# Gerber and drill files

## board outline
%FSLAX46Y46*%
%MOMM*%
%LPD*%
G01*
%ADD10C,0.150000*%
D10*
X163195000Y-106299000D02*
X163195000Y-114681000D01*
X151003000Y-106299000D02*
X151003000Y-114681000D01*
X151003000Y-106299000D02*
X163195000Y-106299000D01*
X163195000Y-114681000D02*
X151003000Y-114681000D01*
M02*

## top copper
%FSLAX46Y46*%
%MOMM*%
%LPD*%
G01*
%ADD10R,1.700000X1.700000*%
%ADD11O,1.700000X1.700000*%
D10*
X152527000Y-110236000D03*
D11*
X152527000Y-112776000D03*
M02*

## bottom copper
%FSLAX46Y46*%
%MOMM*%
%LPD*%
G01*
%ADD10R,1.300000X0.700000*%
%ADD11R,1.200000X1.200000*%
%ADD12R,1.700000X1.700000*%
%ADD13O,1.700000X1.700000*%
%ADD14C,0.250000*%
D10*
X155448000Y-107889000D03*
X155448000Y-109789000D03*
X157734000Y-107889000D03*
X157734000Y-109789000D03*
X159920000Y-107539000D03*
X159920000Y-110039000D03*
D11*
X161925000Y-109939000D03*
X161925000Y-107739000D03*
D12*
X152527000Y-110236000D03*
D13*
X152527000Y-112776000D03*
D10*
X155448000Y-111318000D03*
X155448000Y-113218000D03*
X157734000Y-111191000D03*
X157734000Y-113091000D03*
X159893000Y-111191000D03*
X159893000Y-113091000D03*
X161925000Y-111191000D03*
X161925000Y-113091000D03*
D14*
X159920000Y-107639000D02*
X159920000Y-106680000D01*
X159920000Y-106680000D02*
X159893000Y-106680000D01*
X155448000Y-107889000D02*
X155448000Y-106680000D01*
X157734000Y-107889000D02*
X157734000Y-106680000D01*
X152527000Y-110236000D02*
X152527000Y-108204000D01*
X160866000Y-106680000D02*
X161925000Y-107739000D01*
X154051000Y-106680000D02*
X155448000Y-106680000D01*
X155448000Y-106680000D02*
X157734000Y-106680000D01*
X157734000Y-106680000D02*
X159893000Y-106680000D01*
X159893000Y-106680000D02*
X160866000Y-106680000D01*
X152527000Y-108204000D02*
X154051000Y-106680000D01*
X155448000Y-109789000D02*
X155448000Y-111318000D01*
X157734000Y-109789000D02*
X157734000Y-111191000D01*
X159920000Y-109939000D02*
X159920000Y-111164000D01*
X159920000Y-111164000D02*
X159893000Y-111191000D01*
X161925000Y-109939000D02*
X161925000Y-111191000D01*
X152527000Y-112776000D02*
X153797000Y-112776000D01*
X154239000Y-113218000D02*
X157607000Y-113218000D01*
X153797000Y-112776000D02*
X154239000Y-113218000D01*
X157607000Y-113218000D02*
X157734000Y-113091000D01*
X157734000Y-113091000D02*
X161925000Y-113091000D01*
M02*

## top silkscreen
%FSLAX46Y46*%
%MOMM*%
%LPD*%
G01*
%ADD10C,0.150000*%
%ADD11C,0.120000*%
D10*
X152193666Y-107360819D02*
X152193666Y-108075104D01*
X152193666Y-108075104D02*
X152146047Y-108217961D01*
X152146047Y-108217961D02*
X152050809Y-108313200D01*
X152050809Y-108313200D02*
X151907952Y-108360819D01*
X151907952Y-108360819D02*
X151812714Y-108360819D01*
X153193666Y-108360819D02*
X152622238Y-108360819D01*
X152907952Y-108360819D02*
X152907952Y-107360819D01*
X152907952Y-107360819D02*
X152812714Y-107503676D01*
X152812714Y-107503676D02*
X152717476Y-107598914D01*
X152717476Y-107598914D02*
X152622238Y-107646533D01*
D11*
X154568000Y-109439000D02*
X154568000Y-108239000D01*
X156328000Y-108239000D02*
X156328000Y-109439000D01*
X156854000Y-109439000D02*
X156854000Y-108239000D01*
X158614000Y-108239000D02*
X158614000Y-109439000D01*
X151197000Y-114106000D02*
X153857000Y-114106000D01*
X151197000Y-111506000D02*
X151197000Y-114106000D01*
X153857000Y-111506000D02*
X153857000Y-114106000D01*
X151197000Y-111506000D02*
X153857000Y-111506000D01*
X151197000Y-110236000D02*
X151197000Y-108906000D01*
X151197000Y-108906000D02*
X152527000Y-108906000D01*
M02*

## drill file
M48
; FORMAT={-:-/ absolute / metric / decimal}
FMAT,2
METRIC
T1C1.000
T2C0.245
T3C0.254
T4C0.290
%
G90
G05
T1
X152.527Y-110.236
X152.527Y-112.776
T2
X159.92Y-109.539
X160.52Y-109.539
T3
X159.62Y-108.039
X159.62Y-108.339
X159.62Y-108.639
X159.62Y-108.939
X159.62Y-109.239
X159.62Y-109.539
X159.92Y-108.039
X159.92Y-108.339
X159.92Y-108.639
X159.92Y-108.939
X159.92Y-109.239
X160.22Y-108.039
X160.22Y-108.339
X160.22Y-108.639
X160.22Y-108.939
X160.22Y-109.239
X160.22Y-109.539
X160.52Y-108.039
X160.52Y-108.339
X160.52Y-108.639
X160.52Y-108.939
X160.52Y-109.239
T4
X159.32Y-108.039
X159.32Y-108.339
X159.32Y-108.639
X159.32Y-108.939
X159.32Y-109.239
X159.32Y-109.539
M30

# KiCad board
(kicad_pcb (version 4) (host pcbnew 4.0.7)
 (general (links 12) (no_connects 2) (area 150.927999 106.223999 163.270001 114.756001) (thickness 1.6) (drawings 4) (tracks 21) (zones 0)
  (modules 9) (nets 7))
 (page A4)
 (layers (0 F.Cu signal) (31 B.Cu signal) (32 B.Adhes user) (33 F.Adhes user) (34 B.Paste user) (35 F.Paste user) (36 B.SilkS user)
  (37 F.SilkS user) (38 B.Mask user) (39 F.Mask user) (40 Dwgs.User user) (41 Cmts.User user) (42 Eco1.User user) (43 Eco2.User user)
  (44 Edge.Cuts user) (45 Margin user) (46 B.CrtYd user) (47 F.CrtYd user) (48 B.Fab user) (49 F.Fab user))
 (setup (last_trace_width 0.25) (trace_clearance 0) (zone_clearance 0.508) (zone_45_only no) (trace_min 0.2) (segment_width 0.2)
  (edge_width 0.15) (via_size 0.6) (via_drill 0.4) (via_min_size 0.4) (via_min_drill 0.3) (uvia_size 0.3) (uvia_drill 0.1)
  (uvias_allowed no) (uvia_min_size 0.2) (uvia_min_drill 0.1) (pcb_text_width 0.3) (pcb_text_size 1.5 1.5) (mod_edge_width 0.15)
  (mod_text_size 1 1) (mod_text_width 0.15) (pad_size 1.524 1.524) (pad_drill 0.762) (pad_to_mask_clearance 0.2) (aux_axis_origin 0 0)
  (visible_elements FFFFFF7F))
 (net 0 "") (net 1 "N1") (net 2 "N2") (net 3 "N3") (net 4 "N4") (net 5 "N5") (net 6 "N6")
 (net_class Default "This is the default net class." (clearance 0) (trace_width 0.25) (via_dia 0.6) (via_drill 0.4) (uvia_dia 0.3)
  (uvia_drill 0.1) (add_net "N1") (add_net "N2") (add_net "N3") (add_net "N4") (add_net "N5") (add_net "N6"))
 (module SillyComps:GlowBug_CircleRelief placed (layer F.Cu) (at 155.448 108.839 270)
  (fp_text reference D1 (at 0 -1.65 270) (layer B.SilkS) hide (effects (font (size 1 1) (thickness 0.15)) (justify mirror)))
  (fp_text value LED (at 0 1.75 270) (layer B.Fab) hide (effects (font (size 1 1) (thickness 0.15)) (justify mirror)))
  (fp_line (start 0.6 0.88) (end -0.6 0.88) (layer F.SilkS) (width 0.12))
  (fp_line (start -0.6 -0.88) (end 0.6 -0.88) (layer F.SilkS) (width 0.12))
  (pad 1 smd rect (at -0.95 0 270) (size 0.7 1.3) (layers B.Cu F.Paste B.Mask) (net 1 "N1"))
  (pad 2 smd rect (at 0.95 0 270) (size 0.7 1.3) (layers B.Cu B.Paste B.Mask) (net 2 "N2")))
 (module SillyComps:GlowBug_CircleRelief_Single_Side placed (layer F.Cu) (at 157.734 108.839 270)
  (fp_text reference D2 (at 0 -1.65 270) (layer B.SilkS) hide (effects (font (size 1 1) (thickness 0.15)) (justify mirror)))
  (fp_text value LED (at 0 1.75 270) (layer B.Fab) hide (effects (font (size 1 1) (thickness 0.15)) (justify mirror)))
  (fp_line (start 0.6 0.88) (end -0.6 0.88) (layer F.SilkS) (width 0.12))
  (fp_line (start -0.6 -0.88) (end 0.6 -0.88) (layer F.SilkS) (width 0.12))
  (pad 1 smd rect (at -0.95 0 270) (size 0.7 1.3) (layers B.Cu F.Paste B.Mask) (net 1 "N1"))
  (pad 2 smd rect (at 0.95 0 270) (size 0.7 1.3) (layers B.Cu B.Paste B.Mask) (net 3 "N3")))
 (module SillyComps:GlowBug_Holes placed (layer F.Cu) (at 160.02 108.839 270)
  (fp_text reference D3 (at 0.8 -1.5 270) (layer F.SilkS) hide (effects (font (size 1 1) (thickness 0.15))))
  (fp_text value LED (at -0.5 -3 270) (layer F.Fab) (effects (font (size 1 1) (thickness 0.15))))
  (pad "" np_thru_hole circle (at 0.7 0.7 90) (size 0.29 0.29) (drill 0.29) (layers *.Cu *.Mask))
  (pad "" np_thru_hole circle (at 0.7 -0.2 90) (size 0.254 0.254) (drill 0.254) (layers *.Cu *.Mask))
  (pad "" np_thru_hole circle (at 0.4 -0.2 90) (size 0.254 0.254) (drill 0.254) (layers *.Cu *.Mask))
  (pad "" np_thru_hole circle (at 0.1 -0.2 90) (size 0.254 0.254) (drill 0.254) (layers *.Cu *.Mask))
  (pad "" np_thru_hole circle (at -0.2 -0.2 90) (size 0.254 0.254) (drill 0.254) (layers *.Cu *.Mask))
  (pad "" np_thru_hole circle (at -0.5 -0.2 90) (size 0.254 0.254) (drill 0.254) (layers *.Cu *.Mask))
  (pad "" np_thru_hole circle (at -0.8 -0.2 90) (size 0.254 0.254) (drill 0.254) (layers *.Cu *.Mask))
  (pad "" np_thru_hole circle (at 0.7 0.1 90) (size 0.245 0.245) (drill 0.245) (layers *.Cu *.Mask))
  (pad 1 smd rect (at -1.2 0.1 90) (size 0.7 1.3) (drill (offset 0.1 0)) (layers B.Cu B.Paste B.Mask) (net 1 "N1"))
  (pad 2 smd rect (at 1.1 0.1 270) (size 0.7 1.3) (drill oval (offset 0.1 0)) (layers B.Cu B.Paste B.Mask) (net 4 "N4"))
  (pad "" np_thru_hole circle (at 0.7 -0.5 90) (size 0.245 0.245) (drill 0.245) (layers *.Cu *.Mask))
  (pad "" np_thru_hole circle (at 0.7 0.4 90) (size 0.254 0.254) (drill 0.254) (layers *.Cu *.Mask))
  (pad "" np_thru_hole circle (at 0.4 -0.5 90) (size 0.254 0.254) (drill 0.254) (layers *.Cu *.Mask))
  (pad "" np_thru_hole circle (at 0.4 0.1 90) (size 0.254 0.254) (drill 0.254) (layers *.Cu *.Mask))
  (pad "" np_thru_hole circle (at 0.4 0.4 90) (size 0.254 0.254) (drill 0.254) (layers *.Cu *.Mask))
  (pad "" np_thru_hole circle (at 0.1 -0.5 90) (size 0.254 0.254) (drill 0.254) (layers *.Cu *.Mask))
  (pad "" np_thru_hole circle (at 0.1 0.1 90) (size 0.254 0.254) (drill 0.254) (layers *.Cu *.Mask))
  (pad "" np_thru_hole circle (at 0.1 0.4 90) (size 0.254 0.254) (drill 0.254) (layers *.Cu *.Mask))
  (pad "" np_thru_hole circle (at -0.2 -0.5 90) (size 0.254 0.254) (drill 0.254) (layers *.Cu *.Mask))
  (pad "" np_thru_hole circle (at -0.2 0.1 90) (size 0.254 0.254) (drill 0.254) (layers *.Cu *.Mask))
  (pad "" np_thru_hole circle (at -0.2 0.4 90) (size 0.254 0.254) (drill 0.254) (layers *.Cu *.Mask))
  (pad "" np_thru_hole circle (at -0.5 -0.5 90) (size 0.254 0.254) (drill 0.254) (layers *.Cu *.Mask))
  (pad "" np_thru_hole circle (at -0.5 0.1 90) (size 0.254 0.254) (drill 0.254) (layers *.Cu *.Mask))
  (pad "" np_thru_hole circle (at -0.5 0.4 90) (size 0.254 0.254) (drill 0.254) (layers *.Cu *.Mask))
  (pad "" np_thru_hole circle (at -0.8 -0.5 90) (size 0.254 0.254) (drill 0.254) (layers *.Cu *.Mask))
  (pad "" np_thru_hole circle (at -0.8 0.1 90) (size 0.254 0.254) (drill 0.254) (layers *.Cu *.Mask))
  (pad "" np_thru_hole circle (at -0.8 0.4 90) (size 0.254 0.254) (drill 0.254) (layers *.Cu *.Mask))
  (pad "" np_thru_hole circle (at -0.8 0.7 90) (size 0.29 0.29) (drill 0.29) (layers *.Cu *.Mask))
  (pad "" np_thru_hole circle (at -0.5 0.7 90) (size 0.29 0.29) (drill 0.29) (layers *.Cu *.Mask))
  (pad "" np_thru_hole circle (at -0.2 0.7 90) (size 0.29 0.29) (drill 0.29) (layers *.Cu *.Mask))
  (pad "" np_thru_hole circle (at 0.1 0.7 90) (size 0.29 0.29) (drill 0.29) (layers *.Cu *.Mask))
  (pad "" np_thru_hole circle (at 0.4 0.7 90) (size 0.29 0.29) (drill 0.29) (layers *.Cu *.Mask)))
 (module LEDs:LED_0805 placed (layer B.Cu) (at 161.925 108.839 270)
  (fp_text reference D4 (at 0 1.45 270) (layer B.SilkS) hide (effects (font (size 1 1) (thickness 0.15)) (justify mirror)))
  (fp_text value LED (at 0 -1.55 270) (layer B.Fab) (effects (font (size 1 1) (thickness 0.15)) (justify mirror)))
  (pad 2 smd rect (at 1.1 0 90) (size 1.2 1.2) (layers B.Cu B.Paste B.Mask) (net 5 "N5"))
  (pad 1 smd rect (at -1.1 0 90) (size 1.2 1.2) (layers B.Cu B.Paste B.Mask) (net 1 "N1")))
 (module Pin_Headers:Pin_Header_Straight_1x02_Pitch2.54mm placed (layer F.Cu) (at 152.527 110.236)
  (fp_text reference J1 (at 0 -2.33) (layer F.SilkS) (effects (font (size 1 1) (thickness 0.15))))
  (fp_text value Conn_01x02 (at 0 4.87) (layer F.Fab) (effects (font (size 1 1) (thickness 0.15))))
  (fp_line (start -1.33 3.87) (end 1.33 3.87) (layer F.SilkS) (width 0.12))
  (fp_line (start -1.33 1.27) (end -1.33 3.87) (layer F.SilkS) (width 0.12))
  (fp_line (start 1.33 1.27) (end 1.33 3.87) (layer F.SilkS) (width 0.12))
  (fp_line (start -1.33 1.27) (end 1.33 1.27) (layer F.SilkS) (width 0.12))
  (fp_line (start -1.33 0) (end -1.33 -1.33) (layer F.SilkS) (width 0.12))
  (fp_line (start -1.33 -1.33) (end 0 -1.33) (layer F.SilkS) (width 0.12))
  (pad 1 thru_hole rect (at 0 0) (size 1.7 1.7) (drill 1) (layers *.Cu *.Mask) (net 1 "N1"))
  (pad 2 thru_hole oval (at 0 2.54) (size 1.7 1.7) (drill 1) (layers *.Cu *.Mask) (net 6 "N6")))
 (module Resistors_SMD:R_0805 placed (layer B.Cu) (at 155.448 112.268 270)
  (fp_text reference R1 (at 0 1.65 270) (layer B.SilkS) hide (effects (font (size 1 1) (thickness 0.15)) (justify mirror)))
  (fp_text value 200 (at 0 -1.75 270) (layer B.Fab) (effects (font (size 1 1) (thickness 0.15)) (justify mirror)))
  (pad 1 smd rect (at -0.95 0 270) (size 0.7 1.3) (layers B.Cu B.Paste B.Mask) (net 2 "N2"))
  (pad 2 smd rect (at 0.95 0 270) (size 0.7 1.3) (layers B.Cu B.Paste B.Mask) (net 6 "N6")))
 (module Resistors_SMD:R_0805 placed (layer B.Cu) (at 157.734 112.141 270)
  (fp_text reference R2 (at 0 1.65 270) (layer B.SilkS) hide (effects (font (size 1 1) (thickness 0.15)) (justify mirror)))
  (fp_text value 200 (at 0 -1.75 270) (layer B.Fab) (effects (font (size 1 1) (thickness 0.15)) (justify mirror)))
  (pad 1 smd rect (at -0.95 0 270) (size 0.7 1.3) (layers B.Cu B.Paste B.Mask) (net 3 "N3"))
  (pad 2 smd rect (at 0.95 0 270) (size 0.7 1.3) (layers B.Cu B.Paste B.Mask) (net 6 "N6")))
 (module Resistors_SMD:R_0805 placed (layer B.Cu) (at 159.893 112.141 270)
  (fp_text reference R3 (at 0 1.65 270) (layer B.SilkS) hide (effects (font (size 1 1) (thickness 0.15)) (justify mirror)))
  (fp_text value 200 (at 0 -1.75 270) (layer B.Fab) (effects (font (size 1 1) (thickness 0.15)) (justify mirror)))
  (pad 1 smd rect (at -0.95 0 270) (size 0.7 1.3) (layers B.Cu B.Paste B.Mask) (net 4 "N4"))
  (pad 2 smd rect (at 0.95 0 270) (size 0.7 1.3) (layers B.Cu B.Paste B.Mask) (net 6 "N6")))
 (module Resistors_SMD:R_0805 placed (layer B.Cu) (at 161.925 112.141 270)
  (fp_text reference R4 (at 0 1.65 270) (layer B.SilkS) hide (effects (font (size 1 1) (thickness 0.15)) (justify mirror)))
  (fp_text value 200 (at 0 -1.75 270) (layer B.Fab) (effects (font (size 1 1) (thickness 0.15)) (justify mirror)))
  (pad 1 smd rect (at -0.95 0 270) (size 0.7 1.3) (layers B.Cu B.Paste B.Mask) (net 5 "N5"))
  (pad 2 smd rect (at 0.95 0 270) (size 0.7 1.3) (layers B.Cu B.Paste B.Mask) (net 6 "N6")))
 (gr_line (start 163.195 106.299) (end 163.195 114.681) (angle 90) (layer Edge.Cuts) (width 0.15))
 (gr_line (start 151.003 106.299) (end 151.003 114.681) (angle 90) (layer Edge.Cuts) (width 0.15))
 (gr_line (start 151.003 106.299) (end 163.195 106.299) (angle 90) (layer Edge.Cuts) (width 0.15))
 (gr_line (start 163.195 114.681) (end 151.003 114.681) (angle 90) (layer Edge.Cuts) (width 0.15))
 (segment (start 159.92 107.639) (end 159.92 106.68) (width 0.25) (layer B.Cu) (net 1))
 (segment (start 159.92 106.68) (end 159.893 106.68) (width 0.25) (layer B.Cu) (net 1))
 (segment (start 155.448 107.889) (end 155.448 106.68) (width 0.25) (layer B.Cu) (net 1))
 (segment (start 157.734 107.889) (end 157.734 106.68) (width 0.25) (layer B.Cu) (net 1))
 (segment (start 152.527 110.236) (end 152.527 108.204) (width 0.25) (layer B.Cu) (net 1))
 (segment (start 160.866 106.68) (end 161.925 107.739) (width 0.25) (layer B.Cu) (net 1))
 (segment (start 154.051 106.68) (end 155.448 106.68) (width 0.25) (layer B.Cu) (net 1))
 (segment (start 155.448 106.68) (end 157.734 106.68) (width 0.25) (layer B.Cu) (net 1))
 (segment (start 157.734 106.68) (end 159.893 106.68) (width 0.25) (layer B.Cu) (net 1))
 (segment (start 159.893 106.68) (end 160.866 106.68) (width 0.25) (layer B.Cu) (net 1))
 (segment (start 152.527 108.204) (end 154.051 106.68) (width 0.25) (layer B.Cu) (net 1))
 (segment (start 155.448 109.789) (end 155.448 111.318) (width 0.25) (layer B.Cu) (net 2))
 (segment (start 157.734 109.789) (end 157.734 111.191) (width 0.25) (layer B.Cu) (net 3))
 (segment (start 159.92 109.939) (end 159.92 111.164) (width 0.25) (layer B.Cu) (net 4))
 (segment (start 159.92 111.164) (end 159.893 111.191) (width 0.25) (layer B.Cu) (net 4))
 (segment (start 161.925 109.939) (end 161.925 111.191) (width 0.25) (layer B.Cu) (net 5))
 (segment (start 152.527 112.776) (end 153.797 112.776) (width 0.25) (layer B.Cu) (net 6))
 (segment (start 154.239 113.218) (end 157.607 113.218) (width 0.25) (layer B.Cu) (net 6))
 (segment (start 153.797 112.776) (end 154.239 113.218) (width 0.25) (layer B.Cu) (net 6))
 (segment (start 157.607 113.218) (end 157.734 113.091) (width 0.25) (layer B.Cu) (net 6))
 (segment (start 157.734 113.091) (end 161.925 113.091) (width 0.25) (layer B.Cu) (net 6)))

